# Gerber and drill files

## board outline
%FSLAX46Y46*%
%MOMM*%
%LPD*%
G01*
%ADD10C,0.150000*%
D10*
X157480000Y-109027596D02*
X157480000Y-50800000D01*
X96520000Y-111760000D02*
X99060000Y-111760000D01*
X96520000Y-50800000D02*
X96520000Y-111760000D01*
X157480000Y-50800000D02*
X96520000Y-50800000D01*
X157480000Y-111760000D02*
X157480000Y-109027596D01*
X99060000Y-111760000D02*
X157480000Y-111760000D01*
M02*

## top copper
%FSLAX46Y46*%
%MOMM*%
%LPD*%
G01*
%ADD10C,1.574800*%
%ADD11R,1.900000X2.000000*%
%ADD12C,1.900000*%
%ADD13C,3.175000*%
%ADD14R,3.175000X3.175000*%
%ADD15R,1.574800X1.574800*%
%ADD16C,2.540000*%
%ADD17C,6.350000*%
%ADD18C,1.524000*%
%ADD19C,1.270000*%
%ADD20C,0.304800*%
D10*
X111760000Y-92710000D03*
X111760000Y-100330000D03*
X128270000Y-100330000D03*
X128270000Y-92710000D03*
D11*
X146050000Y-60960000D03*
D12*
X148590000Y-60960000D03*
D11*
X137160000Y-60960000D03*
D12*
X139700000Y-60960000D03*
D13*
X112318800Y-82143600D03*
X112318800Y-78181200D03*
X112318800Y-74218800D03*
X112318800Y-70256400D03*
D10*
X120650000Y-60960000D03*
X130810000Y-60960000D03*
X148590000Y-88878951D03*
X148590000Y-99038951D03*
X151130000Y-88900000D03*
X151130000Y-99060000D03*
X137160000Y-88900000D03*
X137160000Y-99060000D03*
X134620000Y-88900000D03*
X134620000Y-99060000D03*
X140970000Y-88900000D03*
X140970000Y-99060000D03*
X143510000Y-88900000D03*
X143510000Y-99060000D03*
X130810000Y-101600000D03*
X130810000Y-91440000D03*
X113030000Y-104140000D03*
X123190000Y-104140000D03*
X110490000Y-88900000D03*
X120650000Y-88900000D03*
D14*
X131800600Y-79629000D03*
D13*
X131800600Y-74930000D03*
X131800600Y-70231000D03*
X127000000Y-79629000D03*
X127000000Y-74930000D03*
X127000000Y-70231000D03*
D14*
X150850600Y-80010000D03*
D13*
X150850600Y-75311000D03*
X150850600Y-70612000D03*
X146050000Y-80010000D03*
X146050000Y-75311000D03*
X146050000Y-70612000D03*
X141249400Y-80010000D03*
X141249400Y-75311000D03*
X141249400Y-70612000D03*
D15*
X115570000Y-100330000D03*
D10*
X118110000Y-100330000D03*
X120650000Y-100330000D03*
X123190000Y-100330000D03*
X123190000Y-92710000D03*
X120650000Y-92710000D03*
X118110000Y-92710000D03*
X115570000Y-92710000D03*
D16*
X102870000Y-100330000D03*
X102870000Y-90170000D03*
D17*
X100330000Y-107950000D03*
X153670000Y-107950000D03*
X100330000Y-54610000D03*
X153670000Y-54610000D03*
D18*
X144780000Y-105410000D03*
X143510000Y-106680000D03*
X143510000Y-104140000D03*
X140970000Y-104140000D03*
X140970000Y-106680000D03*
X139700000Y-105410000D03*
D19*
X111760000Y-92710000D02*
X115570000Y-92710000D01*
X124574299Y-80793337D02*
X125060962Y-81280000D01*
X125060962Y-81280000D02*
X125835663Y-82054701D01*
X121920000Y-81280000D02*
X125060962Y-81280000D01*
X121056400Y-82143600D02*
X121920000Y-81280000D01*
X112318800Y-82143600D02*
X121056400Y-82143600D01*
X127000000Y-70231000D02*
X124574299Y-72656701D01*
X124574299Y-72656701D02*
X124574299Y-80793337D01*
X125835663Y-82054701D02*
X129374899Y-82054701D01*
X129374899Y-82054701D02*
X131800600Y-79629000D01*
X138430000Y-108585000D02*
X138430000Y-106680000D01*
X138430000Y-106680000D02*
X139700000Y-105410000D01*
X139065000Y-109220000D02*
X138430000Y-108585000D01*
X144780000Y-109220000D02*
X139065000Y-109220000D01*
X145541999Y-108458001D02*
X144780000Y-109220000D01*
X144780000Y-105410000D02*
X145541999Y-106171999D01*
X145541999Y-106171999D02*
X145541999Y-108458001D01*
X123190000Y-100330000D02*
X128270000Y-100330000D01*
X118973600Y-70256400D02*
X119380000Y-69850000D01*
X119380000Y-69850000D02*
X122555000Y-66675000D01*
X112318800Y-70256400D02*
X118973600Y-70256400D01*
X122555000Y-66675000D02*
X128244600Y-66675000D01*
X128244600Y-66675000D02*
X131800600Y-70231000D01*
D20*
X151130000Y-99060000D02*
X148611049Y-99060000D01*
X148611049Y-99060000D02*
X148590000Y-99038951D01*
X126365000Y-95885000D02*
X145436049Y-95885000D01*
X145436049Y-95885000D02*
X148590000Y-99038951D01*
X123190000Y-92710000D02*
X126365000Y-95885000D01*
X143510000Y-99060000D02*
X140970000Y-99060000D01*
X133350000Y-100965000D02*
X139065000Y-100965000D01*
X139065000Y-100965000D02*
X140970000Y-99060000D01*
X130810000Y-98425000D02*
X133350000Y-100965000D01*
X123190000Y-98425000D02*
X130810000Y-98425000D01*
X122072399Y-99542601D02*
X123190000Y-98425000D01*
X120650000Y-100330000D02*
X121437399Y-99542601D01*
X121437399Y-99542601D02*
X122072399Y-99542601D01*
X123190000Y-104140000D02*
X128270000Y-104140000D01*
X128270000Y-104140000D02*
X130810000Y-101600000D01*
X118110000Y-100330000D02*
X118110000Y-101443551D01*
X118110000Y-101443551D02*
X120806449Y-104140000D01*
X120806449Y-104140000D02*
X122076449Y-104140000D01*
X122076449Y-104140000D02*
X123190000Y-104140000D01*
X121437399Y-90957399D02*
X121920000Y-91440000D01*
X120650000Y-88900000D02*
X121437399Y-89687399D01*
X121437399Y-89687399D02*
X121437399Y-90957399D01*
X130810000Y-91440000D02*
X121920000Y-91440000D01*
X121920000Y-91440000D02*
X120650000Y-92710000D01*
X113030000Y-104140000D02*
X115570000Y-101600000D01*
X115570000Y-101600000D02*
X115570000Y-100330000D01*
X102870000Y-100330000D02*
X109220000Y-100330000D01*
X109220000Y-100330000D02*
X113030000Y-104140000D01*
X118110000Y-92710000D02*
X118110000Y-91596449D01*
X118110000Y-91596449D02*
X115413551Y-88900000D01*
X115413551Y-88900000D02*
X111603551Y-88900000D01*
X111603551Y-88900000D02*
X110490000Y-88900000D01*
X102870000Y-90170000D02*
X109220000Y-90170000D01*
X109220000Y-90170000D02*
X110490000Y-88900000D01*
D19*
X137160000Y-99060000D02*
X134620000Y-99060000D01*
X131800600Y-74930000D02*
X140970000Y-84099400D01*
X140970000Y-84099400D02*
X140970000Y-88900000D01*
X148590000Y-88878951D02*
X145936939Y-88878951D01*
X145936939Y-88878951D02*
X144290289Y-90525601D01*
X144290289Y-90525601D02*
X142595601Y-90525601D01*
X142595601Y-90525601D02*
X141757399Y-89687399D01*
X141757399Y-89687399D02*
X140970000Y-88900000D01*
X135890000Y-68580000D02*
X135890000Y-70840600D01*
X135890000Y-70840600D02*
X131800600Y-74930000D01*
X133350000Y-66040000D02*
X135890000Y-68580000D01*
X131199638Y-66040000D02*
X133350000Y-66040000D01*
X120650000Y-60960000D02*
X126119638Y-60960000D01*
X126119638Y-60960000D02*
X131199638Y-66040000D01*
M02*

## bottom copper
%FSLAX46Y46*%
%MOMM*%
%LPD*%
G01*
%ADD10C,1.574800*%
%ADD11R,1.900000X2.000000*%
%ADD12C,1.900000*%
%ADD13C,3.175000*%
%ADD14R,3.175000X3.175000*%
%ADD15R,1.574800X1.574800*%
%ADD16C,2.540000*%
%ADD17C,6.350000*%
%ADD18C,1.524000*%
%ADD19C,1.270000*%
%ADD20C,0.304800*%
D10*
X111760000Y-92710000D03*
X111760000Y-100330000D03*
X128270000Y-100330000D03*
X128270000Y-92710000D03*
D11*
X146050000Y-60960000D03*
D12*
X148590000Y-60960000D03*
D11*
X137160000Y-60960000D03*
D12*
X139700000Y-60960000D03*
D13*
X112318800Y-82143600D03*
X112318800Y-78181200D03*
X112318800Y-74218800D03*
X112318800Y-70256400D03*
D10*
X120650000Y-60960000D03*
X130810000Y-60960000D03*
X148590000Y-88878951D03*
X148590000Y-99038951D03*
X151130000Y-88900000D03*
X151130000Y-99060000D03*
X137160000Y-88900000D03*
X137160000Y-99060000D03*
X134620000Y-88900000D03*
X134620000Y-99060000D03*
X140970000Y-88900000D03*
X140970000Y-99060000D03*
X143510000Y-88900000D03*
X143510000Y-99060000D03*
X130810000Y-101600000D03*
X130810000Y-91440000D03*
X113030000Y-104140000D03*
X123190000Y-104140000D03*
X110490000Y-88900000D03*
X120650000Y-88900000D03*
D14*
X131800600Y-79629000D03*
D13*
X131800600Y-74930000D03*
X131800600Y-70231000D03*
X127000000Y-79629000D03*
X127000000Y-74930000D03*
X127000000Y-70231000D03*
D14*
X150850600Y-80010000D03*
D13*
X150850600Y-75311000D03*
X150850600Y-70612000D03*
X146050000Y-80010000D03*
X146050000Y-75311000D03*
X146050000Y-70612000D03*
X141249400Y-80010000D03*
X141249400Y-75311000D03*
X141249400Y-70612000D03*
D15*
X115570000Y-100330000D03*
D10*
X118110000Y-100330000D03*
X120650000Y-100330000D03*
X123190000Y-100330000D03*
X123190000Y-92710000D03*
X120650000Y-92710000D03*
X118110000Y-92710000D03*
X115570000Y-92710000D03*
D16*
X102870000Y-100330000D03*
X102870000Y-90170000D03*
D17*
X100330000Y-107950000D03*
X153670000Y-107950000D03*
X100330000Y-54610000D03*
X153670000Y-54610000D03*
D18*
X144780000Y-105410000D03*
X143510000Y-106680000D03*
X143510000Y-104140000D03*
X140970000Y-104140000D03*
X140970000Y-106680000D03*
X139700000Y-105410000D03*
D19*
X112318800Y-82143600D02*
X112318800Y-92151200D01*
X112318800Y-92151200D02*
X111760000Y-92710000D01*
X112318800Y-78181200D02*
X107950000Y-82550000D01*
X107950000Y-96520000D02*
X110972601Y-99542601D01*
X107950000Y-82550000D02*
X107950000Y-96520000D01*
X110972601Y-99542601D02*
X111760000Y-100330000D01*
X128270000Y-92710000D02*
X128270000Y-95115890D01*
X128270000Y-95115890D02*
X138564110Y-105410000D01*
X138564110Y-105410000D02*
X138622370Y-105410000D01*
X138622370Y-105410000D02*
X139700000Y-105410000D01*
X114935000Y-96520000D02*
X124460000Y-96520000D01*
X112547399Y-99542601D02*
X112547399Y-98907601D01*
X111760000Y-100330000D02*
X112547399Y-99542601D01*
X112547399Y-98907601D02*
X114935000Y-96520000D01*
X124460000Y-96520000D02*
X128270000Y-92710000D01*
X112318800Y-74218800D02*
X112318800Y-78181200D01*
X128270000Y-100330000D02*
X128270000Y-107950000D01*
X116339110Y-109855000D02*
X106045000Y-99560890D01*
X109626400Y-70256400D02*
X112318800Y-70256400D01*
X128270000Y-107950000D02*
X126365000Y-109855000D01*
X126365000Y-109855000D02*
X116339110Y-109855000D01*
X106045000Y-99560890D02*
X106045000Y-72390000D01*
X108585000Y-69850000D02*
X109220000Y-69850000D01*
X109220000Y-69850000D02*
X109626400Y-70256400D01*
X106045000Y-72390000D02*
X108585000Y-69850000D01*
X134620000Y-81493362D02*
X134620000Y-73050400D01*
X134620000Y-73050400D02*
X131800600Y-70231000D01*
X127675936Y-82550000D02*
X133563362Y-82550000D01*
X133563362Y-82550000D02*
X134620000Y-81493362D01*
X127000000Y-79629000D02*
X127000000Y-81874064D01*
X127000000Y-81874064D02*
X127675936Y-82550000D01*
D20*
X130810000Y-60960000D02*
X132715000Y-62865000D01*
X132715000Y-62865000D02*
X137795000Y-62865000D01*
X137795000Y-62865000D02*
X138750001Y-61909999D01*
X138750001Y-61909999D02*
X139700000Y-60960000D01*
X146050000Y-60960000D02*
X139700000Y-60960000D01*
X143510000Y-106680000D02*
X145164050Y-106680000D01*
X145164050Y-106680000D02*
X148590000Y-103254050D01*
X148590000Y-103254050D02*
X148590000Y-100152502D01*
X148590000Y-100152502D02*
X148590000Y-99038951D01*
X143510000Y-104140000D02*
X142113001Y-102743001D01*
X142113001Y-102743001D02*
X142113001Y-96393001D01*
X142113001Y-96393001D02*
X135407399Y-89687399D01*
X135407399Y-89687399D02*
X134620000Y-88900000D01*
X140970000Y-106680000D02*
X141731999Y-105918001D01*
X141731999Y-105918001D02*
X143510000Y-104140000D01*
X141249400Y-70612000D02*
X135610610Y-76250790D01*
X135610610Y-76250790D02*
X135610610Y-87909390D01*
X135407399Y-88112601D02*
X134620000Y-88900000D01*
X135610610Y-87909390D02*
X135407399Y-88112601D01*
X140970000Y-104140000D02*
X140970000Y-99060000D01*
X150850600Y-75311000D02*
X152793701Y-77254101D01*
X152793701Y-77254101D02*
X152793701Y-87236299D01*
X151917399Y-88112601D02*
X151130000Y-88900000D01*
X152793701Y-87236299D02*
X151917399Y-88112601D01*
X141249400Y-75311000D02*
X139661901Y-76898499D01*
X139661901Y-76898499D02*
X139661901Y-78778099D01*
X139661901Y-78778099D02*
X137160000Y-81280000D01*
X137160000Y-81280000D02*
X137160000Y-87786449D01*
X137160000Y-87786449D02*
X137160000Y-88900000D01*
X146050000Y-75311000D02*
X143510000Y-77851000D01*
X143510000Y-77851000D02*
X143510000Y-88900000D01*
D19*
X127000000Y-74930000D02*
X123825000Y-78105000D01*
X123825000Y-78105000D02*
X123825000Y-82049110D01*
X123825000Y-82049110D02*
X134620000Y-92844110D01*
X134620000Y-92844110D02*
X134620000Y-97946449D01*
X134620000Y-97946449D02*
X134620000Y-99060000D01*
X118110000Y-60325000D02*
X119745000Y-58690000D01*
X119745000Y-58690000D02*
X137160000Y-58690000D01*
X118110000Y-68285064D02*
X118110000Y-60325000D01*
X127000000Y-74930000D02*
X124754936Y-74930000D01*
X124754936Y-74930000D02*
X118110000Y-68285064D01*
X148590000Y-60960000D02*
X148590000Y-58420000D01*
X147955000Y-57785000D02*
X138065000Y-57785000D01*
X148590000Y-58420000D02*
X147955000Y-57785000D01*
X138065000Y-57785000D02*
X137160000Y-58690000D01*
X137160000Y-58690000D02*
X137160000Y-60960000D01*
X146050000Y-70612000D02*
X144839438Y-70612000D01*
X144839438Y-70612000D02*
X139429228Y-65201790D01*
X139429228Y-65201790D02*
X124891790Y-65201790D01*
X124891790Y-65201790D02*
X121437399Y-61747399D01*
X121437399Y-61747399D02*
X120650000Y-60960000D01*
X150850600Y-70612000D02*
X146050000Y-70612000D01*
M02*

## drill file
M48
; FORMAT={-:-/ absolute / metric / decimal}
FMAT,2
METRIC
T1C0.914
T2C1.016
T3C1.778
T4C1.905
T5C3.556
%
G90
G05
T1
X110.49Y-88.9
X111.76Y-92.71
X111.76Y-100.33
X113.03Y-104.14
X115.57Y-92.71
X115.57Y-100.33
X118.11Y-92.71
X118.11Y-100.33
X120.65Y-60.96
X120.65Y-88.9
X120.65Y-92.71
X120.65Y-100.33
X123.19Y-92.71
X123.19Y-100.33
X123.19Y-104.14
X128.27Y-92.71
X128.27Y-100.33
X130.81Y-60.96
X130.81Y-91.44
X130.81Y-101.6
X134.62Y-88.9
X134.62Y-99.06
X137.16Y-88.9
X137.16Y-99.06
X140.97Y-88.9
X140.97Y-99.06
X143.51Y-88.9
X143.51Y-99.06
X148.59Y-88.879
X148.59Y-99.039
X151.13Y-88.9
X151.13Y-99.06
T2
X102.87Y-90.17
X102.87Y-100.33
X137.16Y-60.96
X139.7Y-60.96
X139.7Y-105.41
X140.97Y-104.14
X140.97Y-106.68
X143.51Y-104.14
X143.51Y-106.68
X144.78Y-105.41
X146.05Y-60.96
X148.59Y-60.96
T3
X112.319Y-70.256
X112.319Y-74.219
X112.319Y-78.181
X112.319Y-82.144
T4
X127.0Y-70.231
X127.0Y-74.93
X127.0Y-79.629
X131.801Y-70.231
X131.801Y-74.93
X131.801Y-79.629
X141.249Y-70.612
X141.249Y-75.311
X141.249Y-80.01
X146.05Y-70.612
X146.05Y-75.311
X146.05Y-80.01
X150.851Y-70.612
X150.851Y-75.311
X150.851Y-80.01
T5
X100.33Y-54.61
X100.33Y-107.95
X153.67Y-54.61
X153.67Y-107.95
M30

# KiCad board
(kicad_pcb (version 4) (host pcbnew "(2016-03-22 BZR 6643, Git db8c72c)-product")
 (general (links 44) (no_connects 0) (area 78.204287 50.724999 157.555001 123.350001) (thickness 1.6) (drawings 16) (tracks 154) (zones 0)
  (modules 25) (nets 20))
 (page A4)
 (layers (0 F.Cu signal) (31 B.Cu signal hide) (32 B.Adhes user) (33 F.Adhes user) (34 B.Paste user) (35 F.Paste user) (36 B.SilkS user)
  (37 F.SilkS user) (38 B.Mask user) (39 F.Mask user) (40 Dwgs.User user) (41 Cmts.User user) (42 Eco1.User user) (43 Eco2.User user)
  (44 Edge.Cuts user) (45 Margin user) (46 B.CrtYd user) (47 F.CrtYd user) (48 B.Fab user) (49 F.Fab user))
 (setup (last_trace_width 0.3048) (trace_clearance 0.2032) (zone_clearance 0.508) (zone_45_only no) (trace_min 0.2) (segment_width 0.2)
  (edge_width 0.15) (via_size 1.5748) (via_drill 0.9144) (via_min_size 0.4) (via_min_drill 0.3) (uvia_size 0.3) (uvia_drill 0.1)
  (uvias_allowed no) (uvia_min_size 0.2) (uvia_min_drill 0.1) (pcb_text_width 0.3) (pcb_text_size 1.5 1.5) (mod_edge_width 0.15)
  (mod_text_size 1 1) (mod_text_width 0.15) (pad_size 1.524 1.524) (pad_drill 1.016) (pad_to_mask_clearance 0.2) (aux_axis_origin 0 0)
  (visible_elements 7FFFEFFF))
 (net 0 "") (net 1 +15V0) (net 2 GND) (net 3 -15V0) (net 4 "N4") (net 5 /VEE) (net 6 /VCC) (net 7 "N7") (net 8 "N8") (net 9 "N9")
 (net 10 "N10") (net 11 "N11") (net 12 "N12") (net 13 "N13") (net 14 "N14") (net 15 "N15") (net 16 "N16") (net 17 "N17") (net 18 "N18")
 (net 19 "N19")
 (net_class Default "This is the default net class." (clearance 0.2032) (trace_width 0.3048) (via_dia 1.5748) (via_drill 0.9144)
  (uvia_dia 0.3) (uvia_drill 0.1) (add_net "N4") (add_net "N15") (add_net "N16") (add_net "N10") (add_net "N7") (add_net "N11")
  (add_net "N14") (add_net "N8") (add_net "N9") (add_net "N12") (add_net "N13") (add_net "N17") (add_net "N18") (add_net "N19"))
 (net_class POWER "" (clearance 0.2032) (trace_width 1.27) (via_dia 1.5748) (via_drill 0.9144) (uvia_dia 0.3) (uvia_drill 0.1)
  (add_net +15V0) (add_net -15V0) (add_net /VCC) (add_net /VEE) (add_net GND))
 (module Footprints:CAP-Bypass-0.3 (layer F.Cu) (at 111.76 96.52 270)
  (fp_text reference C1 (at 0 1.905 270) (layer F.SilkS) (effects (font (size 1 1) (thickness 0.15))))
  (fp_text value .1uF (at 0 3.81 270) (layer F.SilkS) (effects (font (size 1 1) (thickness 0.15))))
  (pad 1 thru_hole circle (at -3.81 0 270) (size 1.5748 1.5748) (drill 0.9144) (layers *.Cu *.Mask F.SilkS) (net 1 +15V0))
  (pad 2 thru_hole circle (at 3.81 0 270) (size 1.5748 1.5748) (drill 0.9144) (layers *.Cu *.Mask F.SilkS) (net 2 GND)))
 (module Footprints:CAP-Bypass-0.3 (layer F.Cu) (at 128.27 96.52 90)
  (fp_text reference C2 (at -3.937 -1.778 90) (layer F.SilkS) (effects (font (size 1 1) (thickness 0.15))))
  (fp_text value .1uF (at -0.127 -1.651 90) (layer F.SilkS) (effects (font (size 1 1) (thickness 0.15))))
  (pad 1 thru_hole circle (at -3.81 0 90) (size 1.5748 1.5748) (drill 0.9144) (layers *.Cu *.Mask F.SilkS) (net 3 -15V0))
  (pad 2 thru_hole circle (at 3.81 0 90) (size 1.5748 1.5748) (drill 0.9144) (layers *.Cu *.Mask F.SilkS) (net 2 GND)))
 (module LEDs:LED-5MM (layer F.Cu) (at 146.05 60.96)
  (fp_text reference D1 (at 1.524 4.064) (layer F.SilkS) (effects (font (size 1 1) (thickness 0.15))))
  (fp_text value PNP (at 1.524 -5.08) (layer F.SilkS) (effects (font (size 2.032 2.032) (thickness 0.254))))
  (pad 1 thru_hole rect (at 0 0 90) (size 2 1.9) (drill 1.016) (layers *.Cu *.Mask F.SilkS) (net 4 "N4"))
  (pad 2 thru_hole circle (at 2.54 0) (size 1.9 1.9) (drill 1.016) (layers *.Cu *.Mask F.SilkS) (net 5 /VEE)))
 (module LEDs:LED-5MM (layer F.Cu) (at 137.16 60.96)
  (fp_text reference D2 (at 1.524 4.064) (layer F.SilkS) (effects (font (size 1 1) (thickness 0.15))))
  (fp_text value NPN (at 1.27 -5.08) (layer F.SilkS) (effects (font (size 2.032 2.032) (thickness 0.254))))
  (pad 1 thru_hole rect (at 0 0 90) (size 2 1.9) (drill 1.016) (layers *.Cu *.Mask F.SilkS) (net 5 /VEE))
  (pad 2 thru_hole circle (at 2.54 0) (size 1.9 1.9) (drill 1.016) (layers *.Cu *.Mask F.SilkS) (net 4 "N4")))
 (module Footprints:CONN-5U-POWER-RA (layer F.Cu) (at 112.3188 76.2 90)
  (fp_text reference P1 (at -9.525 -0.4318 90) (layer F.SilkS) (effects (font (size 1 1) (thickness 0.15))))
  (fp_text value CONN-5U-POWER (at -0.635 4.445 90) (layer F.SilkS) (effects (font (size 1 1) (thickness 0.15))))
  (pad 1 thru_hole circle (at -5.9436 0 90) (size 3.175 3.175) (drill 1.778) (layers *.Cu *.Mask F.SilkS) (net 1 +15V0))
  (pad 2 thru_hole circle (at -1.9812 0 90) (size 3.175 3.175) (drill 1.778) (layers *.Cu *.Mask F.SilkS) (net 2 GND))
  (pad 3 thru_hole circle (at 1.9812 0 90) (size 3.175 3.175) (drill 1.778) (layers *.Cu *.Mask F.SilkS) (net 2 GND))
  (pad 4 thru_hole circle (at 5.9436 0 90) (size 3.175 3.175) (drill 1.778) (layers *.Cu *.Mask F.SilkS) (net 3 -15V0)))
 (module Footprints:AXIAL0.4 (layer F.Cu) (at 125.73 60.96)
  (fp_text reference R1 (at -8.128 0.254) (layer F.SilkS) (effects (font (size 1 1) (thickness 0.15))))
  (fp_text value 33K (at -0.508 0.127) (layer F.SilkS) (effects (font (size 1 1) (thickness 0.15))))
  (pad 1 thru_hole circle (at -5.08 0) (size 1.5748 1.5748) (drill 0.9144) (layers *.Cu *.Mask F.SilkS) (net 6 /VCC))
  (pad 2 thru_hole circle (at 5.08 0) (size 1.5748 1.5748) (drill 0.9144) (layers *.Cu *.Mask F.SilkS) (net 4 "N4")))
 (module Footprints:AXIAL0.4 (layer F.Cu) (at 148.59 93.958951 270)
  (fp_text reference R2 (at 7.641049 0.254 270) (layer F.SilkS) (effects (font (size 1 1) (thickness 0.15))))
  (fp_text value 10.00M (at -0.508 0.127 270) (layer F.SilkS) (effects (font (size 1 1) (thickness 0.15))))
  (pad 1 thru_hole circle (at -5.08 0 270) (size 1.5748 1.5748) (drill 0.9144) (layers *.Cu *.Mask F.SilkS) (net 6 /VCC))
  (pad 2 thru_hole circle (at 5.08 0 270) (size 1.5748 1.5748) (drill 0.9144) (layers *.Cu *.Mask F.SilkS) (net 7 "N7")))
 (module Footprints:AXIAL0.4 (layer F.Cu) (at 151.13 93.98 270)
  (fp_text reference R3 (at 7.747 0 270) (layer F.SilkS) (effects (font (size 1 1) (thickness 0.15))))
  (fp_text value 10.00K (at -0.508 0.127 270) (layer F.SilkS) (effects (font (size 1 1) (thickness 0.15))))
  (pad 1 thru_hole circle (at -5.08 0 270) (size 1.5748 1.5748) (drill 0.9144) (layers *.Cu *.Mask F.SilkS) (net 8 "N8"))
  (pad 2 thru_hole circle (at 5.08 0 270) (size 1.5748 1.5748) (drill 0.9144) (layers *.Cu *.Mask F.SilkS) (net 7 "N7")))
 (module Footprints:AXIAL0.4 (layer F.Cu) (at 137.16 93.98 270)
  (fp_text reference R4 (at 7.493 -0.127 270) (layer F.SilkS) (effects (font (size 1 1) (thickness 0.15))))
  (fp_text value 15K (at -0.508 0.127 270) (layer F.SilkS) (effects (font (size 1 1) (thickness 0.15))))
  (pad 1 thru_hole circle (at -5.08 0 270) (size 1.5748 1.5748) (drill 0.9144) (layers *.Cu *.Mask F.SilkS) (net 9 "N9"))
  (pad 2 thru_hole circle (at 5.08 0 270) (size 1.5748 1.5748) (drill 0.9144) (layers *.Cu *.Mask F.SilkS) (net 5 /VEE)))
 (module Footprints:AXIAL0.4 (layer F.Cu) (at 134.62 93.98 270)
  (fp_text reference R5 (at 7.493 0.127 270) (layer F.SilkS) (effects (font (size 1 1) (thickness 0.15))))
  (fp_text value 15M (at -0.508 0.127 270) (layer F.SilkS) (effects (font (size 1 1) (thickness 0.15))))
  (pad 1 thru_hole circle (at -5.08 0 270) (size 1.5748 1.5748) (drill 0.9144) (layers *.Cu *.Mask F.SilkS) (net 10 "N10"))
  (pad 2 thru_hole circle (at 5.08 0 270) (size 1.5748 1.5748) (drill 0.9144) (layers *.Cu *.Mask F.SilkS) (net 5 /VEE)))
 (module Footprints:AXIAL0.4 (layer F.Cu) (at 140.97 93.98 270)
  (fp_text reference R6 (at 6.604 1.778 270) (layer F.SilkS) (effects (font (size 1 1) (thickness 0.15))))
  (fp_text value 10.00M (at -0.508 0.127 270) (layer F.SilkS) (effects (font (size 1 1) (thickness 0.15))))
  (pad 1 thru_hole circle (at -5.08 0 270) (size 1.5748 1.5748) (drill 0.9144) (layers *.Cu *.Mask F.SilkS) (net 6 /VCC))
  (pad 2 thru_hole circle (at 5.08 0 270) (size 1.5748 1.5748) (drill 0.9144) (layers *.Cu *.Mask F.SilkS) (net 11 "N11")))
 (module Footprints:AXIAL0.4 (layer F.Cu) (at 143.51 93.98 270)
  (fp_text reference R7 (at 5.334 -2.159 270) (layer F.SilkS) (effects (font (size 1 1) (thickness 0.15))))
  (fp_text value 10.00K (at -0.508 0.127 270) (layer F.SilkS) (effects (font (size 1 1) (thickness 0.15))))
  (pad 1 thru_hole circle (at -5.08 0 270) (size 1.5748 1.5748) (drill 0.9144) (layers *.Cu *.Mask F.SilkS) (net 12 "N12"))
  (pad 2 thru_hole circle (at 5.08 0 270) (size 1.5748 1.5748) (drill 0.9144) (layers *.Cu *.Mask F.SilkS) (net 11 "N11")))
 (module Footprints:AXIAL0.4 (layer F.Cu) (at 130.81 96.52 90)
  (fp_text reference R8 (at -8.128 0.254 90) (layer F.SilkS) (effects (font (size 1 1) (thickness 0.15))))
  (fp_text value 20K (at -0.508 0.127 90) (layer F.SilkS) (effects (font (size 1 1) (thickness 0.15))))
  (pad 1 thru_hole circle (at -5.08 0 90) (size 1.5748 1.5748) (drill 0.9144) (layers *.Cu *.Mask F.SilkS) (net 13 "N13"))
  (pad 2 thru_hole circle (at 5.08 0 90) (size 1.5748 1.5748) (drill 0.9144) (layers *.Cu *.Mask F.SilkS) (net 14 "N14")))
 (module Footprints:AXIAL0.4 (layer F.Cu) (at 118.11 104.14)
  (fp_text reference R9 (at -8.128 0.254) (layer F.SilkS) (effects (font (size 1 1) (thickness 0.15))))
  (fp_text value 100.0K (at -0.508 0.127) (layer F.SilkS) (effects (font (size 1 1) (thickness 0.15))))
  (pad 1 thru_hole circle (at -5.08 0) (size 1.5748 1.5748) (drill 0.9144) (layers *.Cu *.Mask F.SilkS) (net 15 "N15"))
  (pad 2 thru_hole circle (at 5.08 0) (size 1.5748 1.5748) (drill 0.9144) (layers *.Cu *.Mask F.SilkS) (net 13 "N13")))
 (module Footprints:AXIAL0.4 (layer F.Cu) (at 115.57 88.9)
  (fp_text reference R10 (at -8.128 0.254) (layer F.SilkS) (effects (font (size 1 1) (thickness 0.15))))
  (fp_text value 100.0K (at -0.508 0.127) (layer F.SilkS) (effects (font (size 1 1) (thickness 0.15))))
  (pad 1 thru_hole circle (at -5.08 0) (size 1.5748 1.5748) (drill 0.9144) (layers *.Cu *.Mask F.SilkS) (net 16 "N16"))
  (pad 2 thru_hole circle (at 5.08 0) (size 1.5748 1.5748) (drill 0.9144) (layers *.Cu *.Mask F.SilkS) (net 14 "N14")))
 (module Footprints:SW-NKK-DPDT (layer F.Cu) (at 131.8006 74.93 90)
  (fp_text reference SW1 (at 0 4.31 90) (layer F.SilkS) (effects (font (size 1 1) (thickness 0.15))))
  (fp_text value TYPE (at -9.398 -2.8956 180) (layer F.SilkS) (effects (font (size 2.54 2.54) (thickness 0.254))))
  (pad 1 thru_hole rect (at -4.699 0 90) (size 3.175 3.175) (drill 1.905) (layers *.Cu *.Mask F.SilkS) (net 1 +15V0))
  (pad 2 thru_hole circle (at 0 0 90) (size 3.175 3.175) (drill 1.905) (layers *.Cu *.Mask F.SilkS) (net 6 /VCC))
  (pad 3 thru_hole circle (at 4.699 0 90) (size 3.175 3.175) (drill 1.905) (layers *.Cu *.Mask F.SilkS) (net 3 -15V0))
  (pad 4 thru_hole circle (at -4.699 -4.8006 90) (size 3.175 3.175) (drill 1.905) (layers *.Cu *.Mask F.SilkS) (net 3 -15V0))
  (pad 5 thru_hole circle (at 0 -4.8006 90) (size 3.175 3.175) (drill 1.905) (layers *.Cu *.Mask F.SilkS) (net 5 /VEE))
  (pad 6 thru_hole circle (at 4.699 -4.8006 90) (size 3.175 3.175) (drill 1.905) (layers *.Cu *.Mask F.SilkS) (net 1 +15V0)))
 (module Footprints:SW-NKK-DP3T (layer F.Cu) (at 146.05 75.311 90)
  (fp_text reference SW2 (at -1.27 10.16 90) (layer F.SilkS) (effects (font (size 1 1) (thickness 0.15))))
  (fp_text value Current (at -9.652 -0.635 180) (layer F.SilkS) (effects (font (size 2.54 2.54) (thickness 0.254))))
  (pad 1 thru_hole rect (at -4.699 4.8006 90) (size 3.175 3.175) (drill 1.905) (layers *.Cu *.Mask F.SilkS) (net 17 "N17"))
  (pad 2 thru_hole circle (at 0 4.8006 90) (size 3.175 3.175) (drill 1.905) (layers *.Cu *.Mask F.SilkS) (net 8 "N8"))
  (pad 3 thru_hole circle (at 4.699 4.8006 90) (size 3.175 3.175) (drill 1.905) (layers *.Cu *.Mask F.SilkS) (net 6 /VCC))
  (pad 4 thru_hole circle (at -4.699 0 90) (size 3.175 3.175) (drill 1.905) (layers *.Cu *.Mask F.SilkS) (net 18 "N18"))
  (pad 5 thru_hole circle (at 0 0 90) (size 3.175 3.175) (drill 1.905) (layers *.Cu *.Mask F.SilkS) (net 12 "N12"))
  (pad 6 thru_hole circle (at 4.699 0 90) (size 3.175 3.175) (drill 1.905) (layers *.Cu *.Mask F.SilkS) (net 6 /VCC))
  (pad 7 thru_hole circle (at -4.699 -4.8006 90) (size 3.175 3.175) (drill 1.905) (layers *.Cu *.Mask F.SilkS) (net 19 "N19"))
  (pad 8 thru_hole circle (at 0 -4.8006 90) (size 3.175 3.175) (drill 1.905) (layers *.Cu *.Mask F.SilkS) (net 9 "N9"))
  (pad 9 thru_hole circle (at 4.699 -4.8006 90) (size 3.175 3.175) (drill 1.905) (layers *.Cu *.Mask F.SilkS) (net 10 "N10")))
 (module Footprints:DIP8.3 (layer F.Cu) (at 119.38 96.52)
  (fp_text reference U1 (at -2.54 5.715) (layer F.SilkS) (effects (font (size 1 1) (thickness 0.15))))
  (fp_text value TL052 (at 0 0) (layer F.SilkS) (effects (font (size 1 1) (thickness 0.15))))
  (pad 1 thru_hole rect (at -3.81 3.81) (size 1.5748 1.5748) (drill 0.9144) (layers *.Cu *.Mask F.SilkS) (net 15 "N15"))
  (pad 2 thru_hole circle (at -1.27 3.81) (size 1.5748 1.5748) (drill 0.9144) (layers *.Cu *.Mask F.SilkS) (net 13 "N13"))
  (pad 3 thru_hole circle (at 1.27 3.81) (size 1.5748 1.5748) (drill 0.9144) (layers *.Cu *.Mask F.SilkS) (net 11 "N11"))
  (pad 4 thru_hole circle (at 3.81 3.81) (size 1.5748 1.5748) (drill 0.9144) (layers *.Cu *.Mask F.SilkS) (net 3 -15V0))
  (pad 5 thru_hole circle (at 3.81 -3.81) (size 1.5748 1.5748) (drill 0.9144) (layers *.Cu *.Mask F.SilkS) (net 7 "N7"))
  (pad 6 thru_hole circle (at 1.27 -3.81) (size 1.5748 1.5748) (drill 0.9144) (layers *.Cu *.Mask F.SilkS) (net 14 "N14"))
  (pad 7 thru_hole circle (at -1.27 -3.81) (size 1.5748 1.5748) (drill 0.9144) (layers *.Cu *.Mask F.SilkS) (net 16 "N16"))
  (pad 8 thru_hole circle (at -3.81 -3.81) (size 1.5748 1.5748) (drill 0.9144) (layers *.Cu *.Mask F.SilkS) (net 1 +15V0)))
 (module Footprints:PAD (layer F.Cu) (at 102.87 102.87)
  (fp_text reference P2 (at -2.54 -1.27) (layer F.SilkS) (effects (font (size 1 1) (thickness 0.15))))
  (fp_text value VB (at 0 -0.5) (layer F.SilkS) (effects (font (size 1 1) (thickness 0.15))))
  (pad 1 thru_hole circle (at 0 -2.54) (size 2.54 2.54) (drill 1.016) (layers *.Cu *.Mask F.SilkS) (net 15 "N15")))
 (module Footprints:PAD (layer F.Cu) (at 102.87 92.71)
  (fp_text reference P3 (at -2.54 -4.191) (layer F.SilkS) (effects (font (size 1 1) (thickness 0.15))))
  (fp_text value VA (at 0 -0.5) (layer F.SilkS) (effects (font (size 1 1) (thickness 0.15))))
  (pad 1 thru_hole circle (at 0 -2.54) (size 2.54 2.54) (drill 1.016) (layers *.Cu *.Mask F.SilkS) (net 16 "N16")))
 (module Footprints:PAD (layer F.Cu) (at 100.33 110.49)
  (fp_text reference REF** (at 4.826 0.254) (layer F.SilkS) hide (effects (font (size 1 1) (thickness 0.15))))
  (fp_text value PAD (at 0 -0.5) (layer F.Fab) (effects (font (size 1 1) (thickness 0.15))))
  (pad 1 thru_hole circle (at 0 -2.54) (size 6.35 6.35) (drill 3.556) (layers *.Cu *.Mask F.SilkS)))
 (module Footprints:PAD (layer F.Cu) (at 153.67 110.49)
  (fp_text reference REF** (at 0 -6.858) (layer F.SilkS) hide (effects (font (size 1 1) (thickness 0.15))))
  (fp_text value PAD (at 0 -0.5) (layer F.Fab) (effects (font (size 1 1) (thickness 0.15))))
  (pad 1 thru_hole circle (at 0 -2.54) (size 6.35 6.35) (drill 3.556) (layers *.Cu *.Mask F.SilkS)))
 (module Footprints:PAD (layer F.Cu) (at 100.33 57.15)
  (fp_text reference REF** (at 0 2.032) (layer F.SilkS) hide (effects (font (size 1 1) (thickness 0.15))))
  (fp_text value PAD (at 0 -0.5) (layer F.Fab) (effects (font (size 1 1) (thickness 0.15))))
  (pad 1 thru_hole circle (at 0 -2.54) (size 6.35 6.35) (drill 3.556) (layers *.Cu *.Mask F.SilkS)))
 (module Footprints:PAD (layer F.Cu) (at 153.67 57.15)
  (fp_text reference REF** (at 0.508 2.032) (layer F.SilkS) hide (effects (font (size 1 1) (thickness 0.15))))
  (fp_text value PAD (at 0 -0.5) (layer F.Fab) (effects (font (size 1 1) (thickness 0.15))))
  (pad 1 thru_hole circle (at 0 -2.54) (size 6.35 6.35) (drill 3.556) (layers *.Cu *.Mask F.SilkS)))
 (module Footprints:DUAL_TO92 (layer F.Cu) (at 142.24 105.41 90)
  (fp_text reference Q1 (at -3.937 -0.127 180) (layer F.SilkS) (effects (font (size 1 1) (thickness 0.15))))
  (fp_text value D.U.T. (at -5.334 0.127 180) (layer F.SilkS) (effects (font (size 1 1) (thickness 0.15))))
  (pad 2 thru_hole circle (at 0 2.54 90) (size 1.524 1.524) (drill 1.016) (layers *.Cu *.Mask F.SilkS) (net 2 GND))
  (pad 3 thru_hole circle (at -1.27 1.27 90) (size 1.524 1.524) (drill 1.016) (layers *.Cu *.Mask F.SilkS) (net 7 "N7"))
  (pad 1 thru_hole circle (at 1.27 1.27 90) (size 1.524 1.524) (drill 1.016) (layers *.Cu *.Mask F.SilkS) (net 10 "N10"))
  (pad 6 thru_hole circle (at 1.27 -1.27 90) (size 1.524 1.524) (drill 1.016) (layers *.Cu *.Mask F.SilkS) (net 11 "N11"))
  (pad 4 thru_hole circle (at -1.27 -1.27 90) (size 1.524 1.524) (drill 1.016) (layers *.Cu *.Mask F.SilkS) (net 10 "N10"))
  (pad 5 thru_hole circle (at 0 -2.54 90) (size 1.524 1.524) (drill 1.016) (layers *.Cu *.Mask F.SilkS) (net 2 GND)))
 (gr_line (start 157.48 109.027596) (end 157.48 50.8) (layer Edge.Cuts) (width 0.15))
 (gr_line (start 96.52 111.76) (end 99.06 111.76) (layer Edge.Cuts) (width 0.15))
 (gr_line (start 96.52 50.8) (end 96.52 111.76) (layer Edge.Cuts) (width 0.15))
 (gr_line (start 157.48 50.8) (end 96.52 50.8) (layer Edge.Cuts) (width 0.15))
 (gr_line (start 157.48 111.76) (end 157.48 109.027596) (layer Edge.Cuts) (width 0.15))
 (gr_line (start 99.06 111.76) (end 157.48 111.76) (layer Edge.Cuts) (width 0.15))
 (segment (start 112.3188 82.1436) (end 112.3188 92.1512) (width 1.27) (layer B.Cu) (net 1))
 (segment (start 112.3188 92.1512) (end 111.76 92.71) (width 1.27) (layer B.Cu) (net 1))
 (segment (start 111.76 92.71) (end 115.57 92.71) (width 1.27) (layer F.Cu) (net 1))
 (segment (start 124.574299 80.793337) (end 125.060962 81.28) (width 1.27) (layer F.Cu) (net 1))
 (segment (start 125.060962 81.28) (end 125.835663 82.054701) (width 1.27) (layer F.Cu) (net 1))
 (segment (start 121.92 81.28) (end 125.060962 81.28) (width 1.27) (layer F.Cu) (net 1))
 (segment (start 121.0564 82.1436) (end 121.92 81.28) (width 1.27) (layer F.Cu) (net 1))
 (segment (start 112.3188 82.1436) (end 121.0564 82.1436) (width 1.27) (layer F.Cu) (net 1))
 (segment (start 127 70.231) (end 124.574299 72.656701) (width 1.27) (layer F.Cu) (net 1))
 (segment (start 124.574299 72.656701) (end 124.574299 80.793337) (width 1.27) (layer F.Cu) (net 1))
 (segment (start 125.835663 82.054701) (end 129.374899 82.054701) (width 1.27) (layer F.Cu) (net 1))
 (segment (start 129.374899 82.054701) (end 131.8006 79.629) (width 1.27) (layer F.Cu) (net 1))
 (segment (start 112.3188 78.1812) (end 107.95 82.55) (width 1.27) (layer B.Cu) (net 2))
 (segment (start 107.95 96.52) (end 110.972601 99.542601) (width 1.27) (layer B.Cu) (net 2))
 (segment (start 107.95 82.55) (end 107.95 96.52) (width 1.27) (layer B.Cu) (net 2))
 (segment (start 110.972601 99.542601) (end 111.76 100.33) (width 1.27) (layer B.Cu) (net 2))
 (segment (start 128.27 92.71) (end 128.27 95.11589) (width 1.27) (layer B.Cu) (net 2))
 (segment (start 128.27 95.11589) (end 138.56411 105.41) (width 1.27) (layer B.Cu) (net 2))
 (segment (start 138.56411 105.41) (end 138.62237 105.41) (width 1.27) (layer B.Cu) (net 2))
 (segment (start 138.62237 105.41) (end 139.7 105.41) (width 1.27) (layer B.Cu) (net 2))
 (segment (start 138.43 108.585) (end 138.43 106.68) (width 1.27) (layer F.Cu) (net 2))
 (segment (start 138.43 106.68) (end 139.7 105.41) (width 1.27) (layer F.Cu) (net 2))
 (segment (start 139.065 109.22) (end 138.43 108.585) (width 1.27) (layer F.Cu) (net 2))
 (segment (start 144.78 109.22) (end 139.065 109.22) (width 1.27) (layer F.Cu) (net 2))
 (segment (start 145.541999 108.458001) (end 144.78 109.22) (width 1.27) (layer F.Cu) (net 2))
 (segment (start 144.78 105.41) (end 145.541999 106.171999) (width 1.27) (layer F.Cu) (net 2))
 (segment (start 145.541999 106.171999) (end 145.541999 108.458001) (width 1.27) (layer F.Cu) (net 2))
 (segment (start 114.935 96.52) (end 124.46 96.52) (width 1.27) (layer B.Cu) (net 2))
 (segment (start 112.547399 99.542601) (end 112.547399 98.907601) (width 1.27) (layer B.Cu) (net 2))
 (segment (start 111.76 100.33) (end 112.547399 99.542601) (width 1.27) (layer B.Cu) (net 2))
 (segment (start 112.547399 98.907601) (end 114.935 96.52) (width 1.27) (layer B.Cu) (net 2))
 (segment (start 124.46 96.52) (end 128.27 92.71) (width 1.27) (layer B.Cu) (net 2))
 (segment (start 112.3188 74.2188) (end 112.3188 78.1812) (width 1.27) (layer B.Cu) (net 2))
 (segment (start 128.27 100.33) (end 128.27 107.95) (width 1.27) (layer B.Cu) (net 3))
 (segment (start 116.33911 109.855) (end 106.045 99.56089) (width 1.27) (layer B.Cu) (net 3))
 (segment (start 109.6264 70.2564) (end 112.3188 70.2564) (width 1.27) (layer B.Cu) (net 3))
 (segment (start 128.27 107.95) (end 126.365 109.855) (width 1.27) (layer B.Cu) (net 3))
 (segment (start 126.365 109.855) (end 116.33911 109.855) (width 1.27) (layer B.Cu) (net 3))
 (segment (start 106.045 99.56089) (end 106.045 72.39) (width 1.27) (layer B.Cu) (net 3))
 (segment (start 108.585 69.85) (end 109.22 69.85) (width 1.27) (layer B.Cu) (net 3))
 (segment (start 109.22 69.85) (end 109.6264 70.2564) (width 1.27) (layer B.Cu) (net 3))
 (segment (start 106.045 72.39) (end 108.585 69.85) (width 1.27) (layer B.Cu) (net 3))
 (segment (start 123.19 100.33) (end 128.27 100.33) (width 1.27) (layer F.Cu) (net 3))
 (segment (start 134.62 81.493362) (end 134.62 73.0504) (width 1.27) (layer B.Cu) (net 3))
 (segment (start 134.62 73.0504) (end 131.8006 70.231) (width 1.27) (layer B.Cu) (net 3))
 (segment (start 127.675936 82.55) (end 133.563362 82.55) (width 1.27) (layer B.Cu) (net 3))
 (segment (start 133.563362 82.55) (end 134.62 81.493362) (width 1.27) (layer B.Cu) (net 3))
 (segment (start 127 79.629) (end 127 81.874064) (width 1.27) (layer B.Cu) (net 3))
 (segment (start 127 81.874064) (end 127.675936 82.55) (width 1.27) (layer B.Cu) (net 3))
 (segment (start 118.9736 70.2564) (end 119.38 69.85) (width 1.27) (layer F.Cu) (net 3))
 (segment (start 119.38 69.85) (end 122.555 66.675) (width 1.27) (layer F.Cu) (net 3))
 (segment (start 112.3188 70.2564) (end 118.9736 70.2564) (width 1.27) (layer F.Cu) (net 3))
 (segment (start 122.555 66.675) (end 128.2446 66.675) (width 1.27) (layer F.Cu) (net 3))
 (segment (start 128.2446 66.675) (end 131.8006 70.231) (width 1.27) (layer F.Cu) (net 3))
 (segment (start 130.81 60.96) (end 132.715 62.865) (width 0.3048) (layer B.Cu) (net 4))
 (segment (start 132.715 62.865) (end 137.795 62.865) (width 0.3048) (layer B.Cu) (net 4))
 (segment (start 137.795 62.865) (end 138.750001 61.909999) (width 0.3048) (layer B.Cu) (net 4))
 (segment (start 138.750001 61.909999) (end 139.7 60.96) (width 0.3048) (layer B.Cu) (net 4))
 (segment (start 146.05 60.96) (end 139.7 60.96) (width 0.3048) (layer B.Cu) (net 4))
 (segment (start 151.13 99.06) (end 148.611049 99.06) (width 0.3048) (layer F.Cu) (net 7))
 (segment (start 148.611049 99.06) (end 148.59 99.038951) (width 0.3048) (layer F.Cu) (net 7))
 (segment (start 126.365 95.885) (end 145.436049 95.885) (width 0.3048) (layer F.Cu) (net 7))
 (segment (start 145.436049 95.885) (end 148.59 99.038951) (width 0.3048) (layer F.Cu) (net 7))
 (segment (start 123.19 92.71) (end 126.365 95.885) (width 0.3048) (layer F.Cu) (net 7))
 (segment (start 143.51 106.68) (end 145.16405 106.68) (width 0.3048) (layer B.Cu) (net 7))
 (segment (start 145.16405 106.68) (end 148.59 103.25405) (width 0.3048) (layer B.Cu) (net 7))
 (segment (start 148.59 103.25405) (end 148.59 100.152502) (width 0.3048) (layer B.Cu) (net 7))
 (segment (start 148.59 100.152502) (end 148.59 99.038951) (width 0.3048) (layer B.Cu) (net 7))
 (segment (start 143.51 104.14) (end 142.113001 102.743001) (width 0.3048) (layer B.Cu) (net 10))
 (segment (start 142.113001 102.743001) (end 142.113001 96.393001) (width 0.3048) (layer B.Cu) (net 10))
 (segment (start 142.113001 96.393001) (end 135.407399 89.687399) (width 0.3048) (layer B.Cu) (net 10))
 (segment (start 135.407399 89.687399) (end 134.62 88.9) (width 0.3048) (layer B.Cu) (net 10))
 (segment (start 140.97 106.68) (end 141.731999 105.918001) (width 0.3048) (layer B.Cu) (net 10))
 (segment (start 141.731999 105.918001) (end 143.51 104.14) (width 0.3048) (layer B.Cu) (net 10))
 (segment (start 141.2494 70.612) (end 135.61061 76.25079) (width 0.3048) (layer B.Cu) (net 10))
 (segment (start 135.61061 76.25079) (end 135.61061 87.90939) (width 0.3048) (layer B.Cu) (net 10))
 (segment (start 135.407399 88.112601) (end 134.62 88.9) (width 0.3048) (layer B.Cu) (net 10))
 (segment (start 135.61061 87.90939) (end 135.407399 88.112601) (width 0.3048) (layer B.Cu) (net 10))
 (segment (start 140.97 104.14) (end 140.97 99.06) (width 0.3048) (layer B.Cu) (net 11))
 (segment (start 143.51 99.06) (end 140.97 99.06) (width 0.3048) (layer F.Cu) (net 11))
 (segment (start 133.35 100.965) (end 139.065 100.965) (width 0.3048) (layer F.Cu) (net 11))
 (segment (start 139.065 100.965) (end 140.97 99.06) (width 0.3048) (layer F.Cu) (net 11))
 (segment (start 130.81 98.425) (end 133.35 100.965) (width 0.3048) (layer F.Cu) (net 11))
 (segment (start 123.19 98.425) (end 130.81 98.425) (width 0.3048) (layer F.Cu) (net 11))
 (segment (start 122.072399 99.542601) (end 123.19 98.425) (width 0.3048) (layer F.Cu) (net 11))
 (segment (start 120.65 100.33) (end 121.437399 99.542601) (width 0.3048) (layer F.Cu) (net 11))
 (segment (start 121.437399 99.542601) (end 122.072399 99.542601) (width 0.3048) (layer F.Cu) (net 11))
 (segment (start 150.8506 75.311) (end 152.793701 77.254101) (width 0.3048) (layer B.Cu) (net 8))
 (segment (start 152.793701 77.254101) (end 152.793701 87.236299) (width 0.3048) (layer B.Cu) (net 8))
 (segment (start 151.917399 88.112601) (end 151.13 88.9) (width 0.3048) (layer B.Cu) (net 8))
 (segment (start 152.793701 87.236299) (end 151.917399 88.112601) (width 0.3048) (layer B.Cu) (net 8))
 (segment (start 141.2494 75.311) (end 139.661901 76.898499) (width 0.3048) (layer B.Cu) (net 9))
 (segment (start 139.661901 76.898499) (end 139.661901 78.778099) (width 0.3048) (layer B.Cu) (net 9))
 (segment (start 139.661901 78.778099) (end 137.16 81.28) (width 0.3048) (layer B.Cu) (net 9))
 (segment (start 137.16 81.28) (end 137.16 87.786449) (width 0.3048) (layer B.Cu) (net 9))
 (segment (start 137.16 87.786449) (end 137.16 88.9) (width 0.3048) (layer B.Cu) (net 9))
 (segment (start 146.05 75.311) (end 143.51 77.851) (width 0.3048) (layer B.Cu) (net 12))
 (segment (start 143.51 77.851) (end 143.51 88.9) (width 0.3048) (layer B.Cu) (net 12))
 (segment (start 123.19 104.14) (end 128.27 104.14) (width 0.3048) (layer F.Cu) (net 13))
 (segment (start 128.27 104.14) (end 130.81 101.6) (width 0.3048) (layer F.Cu) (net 13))
 (segment (start 118.11 100.33) (end 118.11 101.443551) (width 0.3048) (layer F.Cu) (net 13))
 (segment (start 118.11 101.443551) (end 120.806449 104.14) (width 0.3048) (layer F.Cu) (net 13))
 (segment (start 120.806449 104.14) (end 122.076449 104.14) (width 0.3048) (layer F.Cu) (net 13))
 (segment (start 122.076449 104.14) (end 123.19 104.14) (width 0.3048) (layer F.Cu) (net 13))
 (segment (start 121.437399 90.957399) (end 121.92 91.44) (width 0.3048) (layer F.Cu) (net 14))
 (segment (start 120.65 88.9) (end 121.437399 89.687399) (width 0.3048) (layer F.Cu) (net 14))
 (segment (start 121.437399 89.687399) (end 121.437399 90.957399) (width 0.3048) (layer F.Cu) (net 14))
 (segment (start 130.81 91.44) (end 121.92 91.44) (width 0.3048) (layer F.Cu) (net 14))
 (segment (start 121.92 91.44) (end 120.65 92.71) (width 0.3048) (layer F.Cu) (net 14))
 (segment (start 113.03 104.14) (end 115.57 101.6) (width 0.3048) (layer F.Cu) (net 15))
 (segment (start 115.57 101.6) (end 115.57 100.33) (width 0.3048) (layer F.Cu) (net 15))
 (segment (start 102.87 100.33) (end 109.22 100.33) (width 0.3048) (layer F.Cu) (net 15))
 (segment (start 109.22 100.33) (end 113.03 104.14) (width 0.3048) (layer F.Cu) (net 15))
 (segment (start 118.11 92.71) (end 118.11 91.596449) (width 0.3048) (layer F.Cu) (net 16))
 (segment (start 118.11 91.596449) (end 115.413551 88.9) (width 0.3048) (layer F.Cu) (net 16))
 (segment (start 115.413551 88.9) (end 111.603551 88.9) (width 0.3048) (layer F.Cu) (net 16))
 (segment (start 111.603551 88.9) (end 110.49 88.9) (width 0.3048) (layer F.Cu) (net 16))
 (segment (start 102.87 90.17) (end 109.22 90.17) (width 0.3048) (layer F.Cu) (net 16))
 (segment (start 109.22 90.17) (end 110.49 88.9) (width 0.3048) (layer F.Cu) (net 16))
 (segment (start 127 74.93) (end 123.825 78.105) (width 1.27) (layer B.Cu) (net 5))
 (segment (start 123.825 78.105) (end 123.825 82.04911) (width 1.27) (layer B.Cu) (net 5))
 (segment (start 123.825 82.04911) (end 134.62 92.84411) (width 1.27) (layer B.Cu) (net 5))
 (segment (start 134.62 92.84411) (end 134.62 97.946449) (width 1.27) (layer B.Cu) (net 5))
 (segment (start 134.62 97.946449) (end 134.62 99.06) (width 1.27) (layer B.Cu) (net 5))
 (segment (start 137.16 99.06) (end 134.62 99.06) (width 1.27) (layer F.Cu) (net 5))
 (segment (start 118.11 60.325) (end 119.745 58.69) (width 1.27) (layer B.Cu) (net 5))
 (segment (start 119.745 58.69) (end 137.16 58.69) (width 1.27) (layer B.Cu) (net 5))
 (segment (start 118.11 68.285064) (end 118.11 60.325) (width 1.27) (layer B.Cu) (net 5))
 (segment (start 127 74.93) (end 124.754936 74.93) (width 1.27) (layer B.Cu) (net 5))
 (segment (start 124.754936 74.93) (end 118.11 68.285064) (width 1.27) (layer B.Cu) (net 5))
 (segment (start 148.59 60.96) (end 148.59 58.42) (width 1.27) (layer B.Cu) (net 5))
 (segment (start 147.955 57.785) (end 138.065 57.785) (width 1.27) (layer B.Cu) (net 5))
 (segment (start 148.59 58.42) (end 147.955 57.785) (width 1.27) (layer B.Cu) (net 5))
 (segment (start 138.065 57.785) (end 137.16 58.69) (width 1.27) (layer B.Cu) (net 5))
 (segment (start 137.16 58.69) (end 137.16 60.96) (width 1.27) (layer B.Cu) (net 5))
 (segment (start 131.8006 74.93) (end 140.97 84.0994) (width 1.27) (layer F.Cu) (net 6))
 (segment (start 140.97 84.0994) (end 140.97 88.9) (width 1.27) (layer F.Cu) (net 6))
 (segment (start 148.59 88.878951) (end 145.936939 88.878951) (width 1.27) (layer F.Cu) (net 6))
 (segment (start 145.936939 88.878951) (end 144.290289 90.525601) (width 1.27) (layer F.Cu) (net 6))
 (segment (start 144.290289 90.525601) (end 142.595601 90.525601) (width 1.27) (layer F.Cu) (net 6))
 (segment (start 142.595601 90.525601) (end 141.757399 89.687399) (width 1.27) (layer F.Cu) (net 6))
 (segment (start 141.757399 89.687399) (end 140.97 88.9) (width 1.27) (layer F.Cu) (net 6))
 (segment (start 146.05 70.612) (end 144.839438 70.612) (width 1.27) (layer B.Cu) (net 6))
 (segment (start 144.839438 70.612) (end 139.429228 65.20179) (width 1.27) (layer B.Cu) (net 6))
 (segment (start 139.429228 65.20179) (end 124.89179 65.20179) (width 1.27) (layer B.Cu) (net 6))
 (segment (start 124.89179 65.20179) (end 121.437399 61.747399) (width 1.27) (layer B.Cu) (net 6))
 (segment (start 121.437399 61.747399) (end 120.65 60.96) (width 1.27) (layer B.Cu) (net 6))
 (segment (start 150.8506 70.612) (end 146.05 70.612) (width 1.27) (layer B.Cu) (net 6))
 (segment (start 135.89 68.58) (end 135.89 70.8406) (width 1.27) (layer F.Cu) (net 6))
 (segment (start 135.89 70.8406) (end 131.8006 74.93) (width 1.27) (layer F.Cu) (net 6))
 (segment (start 133.35 66.04) (end 135.89 68.58) (width 1.27) (layer F.Cu) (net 6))
 (segment (start 131.199638 66.04) (end 133.35 66.04) (width 1.27) (layer F.Cu) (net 6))
 (segment (start 120.65 60.96) (end 126.119638 60.96) (width 1.27) (layer F.Cu) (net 6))
 (segment (start 126.119638 60.96) (end 131.199638 66.04) (width 1.27) (layer F.Cu) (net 6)))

